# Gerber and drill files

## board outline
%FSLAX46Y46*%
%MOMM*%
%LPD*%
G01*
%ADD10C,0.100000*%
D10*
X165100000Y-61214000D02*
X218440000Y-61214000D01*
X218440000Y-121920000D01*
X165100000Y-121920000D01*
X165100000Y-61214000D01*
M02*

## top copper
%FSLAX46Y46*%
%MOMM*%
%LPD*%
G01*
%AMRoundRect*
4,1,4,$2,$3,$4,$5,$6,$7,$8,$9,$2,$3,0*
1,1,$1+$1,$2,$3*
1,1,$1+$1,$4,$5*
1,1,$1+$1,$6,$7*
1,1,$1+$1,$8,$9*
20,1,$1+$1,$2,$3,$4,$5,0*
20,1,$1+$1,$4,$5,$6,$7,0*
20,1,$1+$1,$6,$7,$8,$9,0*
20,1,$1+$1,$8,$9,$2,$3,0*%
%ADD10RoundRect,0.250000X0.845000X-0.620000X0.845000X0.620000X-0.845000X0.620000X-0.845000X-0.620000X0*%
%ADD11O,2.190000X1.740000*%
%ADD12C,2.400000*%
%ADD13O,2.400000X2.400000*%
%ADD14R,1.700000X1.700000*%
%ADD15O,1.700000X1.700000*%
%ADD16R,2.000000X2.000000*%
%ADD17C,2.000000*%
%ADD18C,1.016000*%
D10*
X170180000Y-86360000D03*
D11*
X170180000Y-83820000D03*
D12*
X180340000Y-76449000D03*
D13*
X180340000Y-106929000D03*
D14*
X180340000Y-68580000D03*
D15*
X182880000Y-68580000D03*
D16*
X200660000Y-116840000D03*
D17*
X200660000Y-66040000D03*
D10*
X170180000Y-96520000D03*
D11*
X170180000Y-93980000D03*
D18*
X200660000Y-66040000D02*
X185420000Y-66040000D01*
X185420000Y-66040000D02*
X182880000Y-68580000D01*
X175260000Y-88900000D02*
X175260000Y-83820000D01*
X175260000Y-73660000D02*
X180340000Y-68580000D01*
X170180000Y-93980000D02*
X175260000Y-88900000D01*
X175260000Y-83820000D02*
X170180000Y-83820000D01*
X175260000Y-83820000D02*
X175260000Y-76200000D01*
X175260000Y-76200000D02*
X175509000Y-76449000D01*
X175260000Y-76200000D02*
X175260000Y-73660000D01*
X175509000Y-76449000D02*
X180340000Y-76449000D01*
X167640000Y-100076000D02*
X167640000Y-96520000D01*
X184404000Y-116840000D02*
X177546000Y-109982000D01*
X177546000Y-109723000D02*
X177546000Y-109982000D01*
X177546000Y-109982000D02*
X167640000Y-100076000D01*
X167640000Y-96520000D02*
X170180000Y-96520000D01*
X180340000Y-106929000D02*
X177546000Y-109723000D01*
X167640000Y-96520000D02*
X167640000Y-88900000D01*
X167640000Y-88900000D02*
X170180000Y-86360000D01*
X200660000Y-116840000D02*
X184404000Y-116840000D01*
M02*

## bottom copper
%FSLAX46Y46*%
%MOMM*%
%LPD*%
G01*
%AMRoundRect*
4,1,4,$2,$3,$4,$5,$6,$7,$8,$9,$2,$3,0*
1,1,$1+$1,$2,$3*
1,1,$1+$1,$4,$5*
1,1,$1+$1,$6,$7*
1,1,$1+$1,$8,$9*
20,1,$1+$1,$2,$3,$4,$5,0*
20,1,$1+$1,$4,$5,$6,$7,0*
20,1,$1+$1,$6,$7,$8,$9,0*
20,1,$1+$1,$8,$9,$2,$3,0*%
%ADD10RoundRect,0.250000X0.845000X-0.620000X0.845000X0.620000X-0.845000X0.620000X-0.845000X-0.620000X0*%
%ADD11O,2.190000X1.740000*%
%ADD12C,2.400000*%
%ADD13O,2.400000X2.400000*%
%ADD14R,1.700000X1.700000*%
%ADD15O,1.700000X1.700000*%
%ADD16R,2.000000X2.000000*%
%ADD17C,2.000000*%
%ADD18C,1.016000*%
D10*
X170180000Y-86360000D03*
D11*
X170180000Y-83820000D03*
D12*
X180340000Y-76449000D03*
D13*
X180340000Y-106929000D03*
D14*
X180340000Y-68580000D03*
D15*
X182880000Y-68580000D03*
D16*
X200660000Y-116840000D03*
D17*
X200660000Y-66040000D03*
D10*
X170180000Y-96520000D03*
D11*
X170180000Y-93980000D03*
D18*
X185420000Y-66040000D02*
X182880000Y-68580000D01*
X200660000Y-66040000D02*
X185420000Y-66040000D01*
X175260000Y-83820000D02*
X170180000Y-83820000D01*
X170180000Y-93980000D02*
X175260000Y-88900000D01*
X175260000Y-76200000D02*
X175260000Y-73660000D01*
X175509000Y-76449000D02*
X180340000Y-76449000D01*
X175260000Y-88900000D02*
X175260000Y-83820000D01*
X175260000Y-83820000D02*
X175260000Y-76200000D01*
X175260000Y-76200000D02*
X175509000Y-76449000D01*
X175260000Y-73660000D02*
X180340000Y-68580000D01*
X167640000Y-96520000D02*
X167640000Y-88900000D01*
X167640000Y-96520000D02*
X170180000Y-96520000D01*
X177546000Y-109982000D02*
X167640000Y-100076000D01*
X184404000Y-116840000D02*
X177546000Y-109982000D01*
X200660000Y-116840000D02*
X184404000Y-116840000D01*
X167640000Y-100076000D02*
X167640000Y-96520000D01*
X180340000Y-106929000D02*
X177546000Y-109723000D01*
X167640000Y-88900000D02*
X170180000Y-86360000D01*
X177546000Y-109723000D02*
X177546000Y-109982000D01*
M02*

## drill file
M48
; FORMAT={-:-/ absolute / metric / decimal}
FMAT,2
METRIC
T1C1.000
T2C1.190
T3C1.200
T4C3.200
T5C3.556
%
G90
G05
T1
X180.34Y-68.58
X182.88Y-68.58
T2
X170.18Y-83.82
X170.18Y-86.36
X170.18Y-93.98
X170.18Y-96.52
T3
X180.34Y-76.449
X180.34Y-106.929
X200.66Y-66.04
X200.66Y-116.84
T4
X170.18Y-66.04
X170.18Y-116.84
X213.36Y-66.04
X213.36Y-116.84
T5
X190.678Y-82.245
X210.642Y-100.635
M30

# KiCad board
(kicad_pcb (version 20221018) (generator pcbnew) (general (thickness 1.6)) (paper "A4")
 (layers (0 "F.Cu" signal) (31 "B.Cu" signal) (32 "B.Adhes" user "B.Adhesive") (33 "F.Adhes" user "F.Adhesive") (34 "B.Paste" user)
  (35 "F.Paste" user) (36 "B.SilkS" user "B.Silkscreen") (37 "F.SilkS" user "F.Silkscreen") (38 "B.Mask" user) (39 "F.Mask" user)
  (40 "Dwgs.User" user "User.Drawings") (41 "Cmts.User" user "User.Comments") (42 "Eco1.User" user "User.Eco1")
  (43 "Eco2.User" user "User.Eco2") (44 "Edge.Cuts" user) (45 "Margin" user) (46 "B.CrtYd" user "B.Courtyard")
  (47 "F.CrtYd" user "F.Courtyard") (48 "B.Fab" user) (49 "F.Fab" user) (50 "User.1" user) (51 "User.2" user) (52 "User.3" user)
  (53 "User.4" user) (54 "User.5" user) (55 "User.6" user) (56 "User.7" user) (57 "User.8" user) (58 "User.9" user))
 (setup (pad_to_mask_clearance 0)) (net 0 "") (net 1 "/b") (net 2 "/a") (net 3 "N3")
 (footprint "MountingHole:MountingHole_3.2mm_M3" (layer "F.Cu") (at 170.18 66.04)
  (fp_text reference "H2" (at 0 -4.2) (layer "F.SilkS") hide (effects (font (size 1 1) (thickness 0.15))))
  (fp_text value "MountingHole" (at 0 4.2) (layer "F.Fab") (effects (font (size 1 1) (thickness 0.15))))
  (pad "" np_thru_hole circle (at 0 0) (size 3.2 3.2) (drill 3.2) (layers "*.Cu" "*.Mask")))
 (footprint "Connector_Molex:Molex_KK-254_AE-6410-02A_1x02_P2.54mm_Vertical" (layer "F.Cu") (at 170.18 86.36 90)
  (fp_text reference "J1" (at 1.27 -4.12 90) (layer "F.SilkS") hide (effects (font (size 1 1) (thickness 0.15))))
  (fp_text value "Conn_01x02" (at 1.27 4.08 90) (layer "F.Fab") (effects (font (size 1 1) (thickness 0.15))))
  (pad "1" thru_hole roundrect (at 0 0 90) (size 1.74 2.19) (drill 1.19) (layers "*.Cu" "*.Mask") (roundrect_rratio 0.1436781609)
   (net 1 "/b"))
  (pad "2" thru_hole oval (at 2.54 0 90) (size 1.74 2.19) (drill 1.19) (layers "*.Cu" "*.Mask") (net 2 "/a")))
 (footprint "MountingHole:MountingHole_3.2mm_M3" (layer "F.Cu") (at 213.36 66.04)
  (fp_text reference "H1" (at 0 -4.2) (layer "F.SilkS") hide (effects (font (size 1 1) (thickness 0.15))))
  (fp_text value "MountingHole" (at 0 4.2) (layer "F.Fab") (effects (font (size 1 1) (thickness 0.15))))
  (pad "" np_thru_hole circle (at 0 0) (size 3.2 3.2) (drill 3.2) (layers "*.Cu" "*.Mask")))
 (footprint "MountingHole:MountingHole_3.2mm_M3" (layer "F.Cu") (at 170.18 116.84)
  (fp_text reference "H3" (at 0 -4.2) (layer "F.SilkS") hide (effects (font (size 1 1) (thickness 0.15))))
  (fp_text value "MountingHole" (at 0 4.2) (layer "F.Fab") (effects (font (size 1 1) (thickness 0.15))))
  (pad "" np_thru_hole circle (at 0 0) (size 3.2 3.2) (drill 3.2) (layers "*.Cu" "*.Mask")))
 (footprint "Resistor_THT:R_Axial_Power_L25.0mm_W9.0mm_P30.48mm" (layer "F.Cu") (at 180.34 76.449 -90)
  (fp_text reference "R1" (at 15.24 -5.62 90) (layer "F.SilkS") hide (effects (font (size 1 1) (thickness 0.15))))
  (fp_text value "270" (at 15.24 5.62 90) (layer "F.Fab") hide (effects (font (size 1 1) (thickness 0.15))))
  (pad "1" thru_hole circle (at 0 0 270) (size 2.4 2.4) (drill 1.2) (layers "*.Cu" "*.Mask") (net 2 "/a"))
  (pad "2" thru_hole oval (at 30.48 0 270) (size 2.4 2.4) (drill 1.2) (layers "*.Cu" "*.Mask") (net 1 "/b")))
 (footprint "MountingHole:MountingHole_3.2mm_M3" (layer "F.Cu") (at 213.36 116.84)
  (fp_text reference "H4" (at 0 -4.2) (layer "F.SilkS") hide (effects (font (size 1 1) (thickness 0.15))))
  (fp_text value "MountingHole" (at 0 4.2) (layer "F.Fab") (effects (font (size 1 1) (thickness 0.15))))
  (pad "" np_thru_hole circle (at 0 0) (size 3.2 3.2) (drill 3.2) (layers "*.Cu" "*.Mask")))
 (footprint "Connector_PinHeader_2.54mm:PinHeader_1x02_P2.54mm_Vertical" (layer "F.Cu") (at 180.34 68.58 90)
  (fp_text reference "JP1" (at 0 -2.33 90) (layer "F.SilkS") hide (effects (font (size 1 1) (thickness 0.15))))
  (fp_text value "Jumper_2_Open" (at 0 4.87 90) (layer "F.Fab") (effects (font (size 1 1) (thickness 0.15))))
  (pad "1" thru_hole rect (at 0 0 90) (size 1.7 1.7) (drill 1) (layers "*.Cu" "*.Mask") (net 2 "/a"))
  (pad "2" thru_hole oval (at 0 2.54 90) (size 1.7 1.7) (drill 1) (layers "*.Cu" "*.Mask") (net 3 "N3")))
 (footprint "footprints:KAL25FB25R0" (layer "F.Cu") (at 200.66 116.84 90)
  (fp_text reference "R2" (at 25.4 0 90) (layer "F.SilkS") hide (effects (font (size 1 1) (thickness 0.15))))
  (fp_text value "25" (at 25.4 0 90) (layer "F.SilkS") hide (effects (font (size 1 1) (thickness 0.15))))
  (pad "" np_thru_hole circle (at 16.2052 9.9822 90) (size 4.064 4.064) (drill 3.556) (layers))
  (pad "" np_thru_hole circle (at 34.5948 -9.9822 90) (size 4.064 4.064) (drill 3.556) (layers))
  (pad "1" thru_hole rect (at 0 0 90) (size 2 2) (drill 1.2) (layers "*.Cu" "*.Mask") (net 1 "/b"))
  (pad "2" thru_hole circle (at 50.8 0 90) (size 2 2) (drill 1.2) (layers "*.Cu" "*.Mask") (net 3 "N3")))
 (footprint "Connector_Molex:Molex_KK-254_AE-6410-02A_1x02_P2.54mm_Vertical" (layer "F.Cu") (at 170.18 96.52 90)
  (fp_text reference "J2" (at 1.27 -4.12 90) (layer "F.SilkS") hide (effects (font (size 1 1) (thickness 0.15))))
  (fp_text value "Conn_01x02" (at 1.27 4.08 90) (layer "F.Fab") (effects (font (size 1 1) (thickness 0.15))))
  (pad "1" thru_hole roundrect (at 0 0 90) (size 1.74 2.19) (drill 1.19) (layers "*.Cu" "*.Mask") (roundrect_rratio 0.1436781609)
   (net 1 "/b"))
  (pad "2" thru_hole oval (at 2.54 0 90) (size 1.74 2.19) (drill 1.19) (layers "*.Cu" "*.Mask") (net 2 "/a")))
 (gr_rect (start 165.1 61.214) (end 218.44 121.92) (stroke (width 0.1) (type default)) (fill none) (layer "Edge.Cuts"))
 (segment (start 200.66 66.04) (end 185.42 66.04) (width 1.016) (layer "F.Cu") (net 3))
 (segment (start 185.42 66.04) (end 182.88 68.58) (width 1.016) (layer "F.Cu") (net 3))
 (segment (start 185.42 66.04) (end 182.88 68.58) (width 1.016) (layer "B.Cu") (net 3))
 (segment (start 200.66 66.04) (end 185.42 66.04) (width 1.016) (layer "B.Cu") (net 3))
 (segment (start 175.26 88.9) (end 175.26 83.82) (width 1.016) (layer "F.Cu") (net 2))
 (segment (start 175.26 73.66) (end 180.34 68.58) (width 1.016) (layer "F.Cu") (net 2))
 (segment (start 170.18 93.98) (end 175.26 88.9) (width 1.016) (layer "F.Cu") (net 2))
 (segment (start 175.26 83.82) (end 170.18 83.82) (width 1.016) (layer "F.Cu") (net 2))
 (segment (start 175.26 83.82) (end 175.26 76.2) (width 1.016) (layer "F.Cu") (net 2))
 (segment (start 175.26 76.2) (end 175.509 76.449) (width 1.016) (layer "F.Cu") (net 2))
 (segment (start 175.26 76.2) (end 175.26 73.66) (width 1.016) (layer "F.Cu") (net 2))
 (segment (start 175.509 76.449) (end 180.34 76.449) (width 1.016) (layer "F.Cu") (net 2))
 (segment (start 175.26 83.82) (end 170.18 83.82) (width 1.016) (layer "B.Cu") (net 2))
 (segment (start 170.18 93.98) (end 175.26 88.9) (width 1.016) (layer "B.Cu") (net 2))
 (segment (start 175.26 76.2) (end 175.26 73.66) (width 1.016) (layer "B.Cu") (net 2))
 (segment (start 175.509 76.449) (end 180.34 76.449) (width 1.016) (layer "B.Cu") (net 2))
 (segment (start 175.26 88.9) (end 175.26 83.82) (width 1.016) (layer "B.Cu") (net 2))
 (segment (start 175.26 83.82) (end 175.26 76.2) (width 1.016) (layer "B.Cu") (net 2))
 (segment (start 175.26 76.2) (end 175.509 76.449) (width 1.016) (layer "B.Cu") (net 2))
 (segment (start 175.26 73.66) (end 180.34 68.58) (width 1.016) (layer "B.Cu") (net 2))
 (segment (start 167.64 100.076) (end 167.64 96.52) (width 1.016) (layer "F.Cu") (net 1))
 (segment (start 184.404 116.84) (end 177.546 109.982) (width 1.016) (layer "F.Cu") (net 1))
 (segment (start 177.546 109.723) (end 177.546 109.982) (width 1.016) (layer "F.Cu") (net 1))
 (segment (start 177.546 109.982) (end 167.64 100.076) (width 1.016) (layer "F.Cu") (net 1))
 (segment (start 167.64 96.52) (end 170.18 96.52) (width 1.016) (layer "F.Cu") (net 1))
 (segment (start 180.34 106.929) (end 177.546 109.723) (width 1.016) (layer "F.Cu") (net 1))
 (segment (start 167.64 96.52) (end 167.64 88.9) (width 1.016) (layer "F.Cu") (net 1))
 (segment (start 167.64 88.9) (end 170.18 86.36) (width 1.016) (layer "F.Cu") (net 1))
 (segment (start 200.66 116.84) (end 184.404 116.84) (width 1.016) (layer "F.Cu") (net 1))
 (segment (start 167.64 96.52) (end 167.64 88.9) (width 1.016) (layer "B.Cu") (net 1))
 (segment (start 167.64 96.52) (end 170.18 96.52) (width 1.016) (layer "B.Cu") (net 1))
 (segment (start 177.546 109.982) (end 167.64 100.076) (width 1.016) (layer "B.Cu") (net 1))
 (segment (start 184.404 116.84) (end 177.546 109.982) (width 1.016) (layer "B.Cu") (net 1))
 (segment (start 200.66 116.84) (end 184.404 116.84) (width 1.016) (layer "B.Cu") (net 1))
 (segment (start 167.64 100.076) (end 167.64 96.52) (width 1.016) (layer "B.Cu") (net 1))
 (segment (start 180.34 106.929) (end 177.546 109.723) (width 1.016) (layer "B.Cu") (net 1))
 (segment (start 167.64 88.9) (end 170.18 86.36) (width 1.016) (layer "B.Cu") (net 1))
 (segment (start 177.546 109.723) (end 177.546 109.982) (width 1.016) (layer "B.Cu") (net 1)))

